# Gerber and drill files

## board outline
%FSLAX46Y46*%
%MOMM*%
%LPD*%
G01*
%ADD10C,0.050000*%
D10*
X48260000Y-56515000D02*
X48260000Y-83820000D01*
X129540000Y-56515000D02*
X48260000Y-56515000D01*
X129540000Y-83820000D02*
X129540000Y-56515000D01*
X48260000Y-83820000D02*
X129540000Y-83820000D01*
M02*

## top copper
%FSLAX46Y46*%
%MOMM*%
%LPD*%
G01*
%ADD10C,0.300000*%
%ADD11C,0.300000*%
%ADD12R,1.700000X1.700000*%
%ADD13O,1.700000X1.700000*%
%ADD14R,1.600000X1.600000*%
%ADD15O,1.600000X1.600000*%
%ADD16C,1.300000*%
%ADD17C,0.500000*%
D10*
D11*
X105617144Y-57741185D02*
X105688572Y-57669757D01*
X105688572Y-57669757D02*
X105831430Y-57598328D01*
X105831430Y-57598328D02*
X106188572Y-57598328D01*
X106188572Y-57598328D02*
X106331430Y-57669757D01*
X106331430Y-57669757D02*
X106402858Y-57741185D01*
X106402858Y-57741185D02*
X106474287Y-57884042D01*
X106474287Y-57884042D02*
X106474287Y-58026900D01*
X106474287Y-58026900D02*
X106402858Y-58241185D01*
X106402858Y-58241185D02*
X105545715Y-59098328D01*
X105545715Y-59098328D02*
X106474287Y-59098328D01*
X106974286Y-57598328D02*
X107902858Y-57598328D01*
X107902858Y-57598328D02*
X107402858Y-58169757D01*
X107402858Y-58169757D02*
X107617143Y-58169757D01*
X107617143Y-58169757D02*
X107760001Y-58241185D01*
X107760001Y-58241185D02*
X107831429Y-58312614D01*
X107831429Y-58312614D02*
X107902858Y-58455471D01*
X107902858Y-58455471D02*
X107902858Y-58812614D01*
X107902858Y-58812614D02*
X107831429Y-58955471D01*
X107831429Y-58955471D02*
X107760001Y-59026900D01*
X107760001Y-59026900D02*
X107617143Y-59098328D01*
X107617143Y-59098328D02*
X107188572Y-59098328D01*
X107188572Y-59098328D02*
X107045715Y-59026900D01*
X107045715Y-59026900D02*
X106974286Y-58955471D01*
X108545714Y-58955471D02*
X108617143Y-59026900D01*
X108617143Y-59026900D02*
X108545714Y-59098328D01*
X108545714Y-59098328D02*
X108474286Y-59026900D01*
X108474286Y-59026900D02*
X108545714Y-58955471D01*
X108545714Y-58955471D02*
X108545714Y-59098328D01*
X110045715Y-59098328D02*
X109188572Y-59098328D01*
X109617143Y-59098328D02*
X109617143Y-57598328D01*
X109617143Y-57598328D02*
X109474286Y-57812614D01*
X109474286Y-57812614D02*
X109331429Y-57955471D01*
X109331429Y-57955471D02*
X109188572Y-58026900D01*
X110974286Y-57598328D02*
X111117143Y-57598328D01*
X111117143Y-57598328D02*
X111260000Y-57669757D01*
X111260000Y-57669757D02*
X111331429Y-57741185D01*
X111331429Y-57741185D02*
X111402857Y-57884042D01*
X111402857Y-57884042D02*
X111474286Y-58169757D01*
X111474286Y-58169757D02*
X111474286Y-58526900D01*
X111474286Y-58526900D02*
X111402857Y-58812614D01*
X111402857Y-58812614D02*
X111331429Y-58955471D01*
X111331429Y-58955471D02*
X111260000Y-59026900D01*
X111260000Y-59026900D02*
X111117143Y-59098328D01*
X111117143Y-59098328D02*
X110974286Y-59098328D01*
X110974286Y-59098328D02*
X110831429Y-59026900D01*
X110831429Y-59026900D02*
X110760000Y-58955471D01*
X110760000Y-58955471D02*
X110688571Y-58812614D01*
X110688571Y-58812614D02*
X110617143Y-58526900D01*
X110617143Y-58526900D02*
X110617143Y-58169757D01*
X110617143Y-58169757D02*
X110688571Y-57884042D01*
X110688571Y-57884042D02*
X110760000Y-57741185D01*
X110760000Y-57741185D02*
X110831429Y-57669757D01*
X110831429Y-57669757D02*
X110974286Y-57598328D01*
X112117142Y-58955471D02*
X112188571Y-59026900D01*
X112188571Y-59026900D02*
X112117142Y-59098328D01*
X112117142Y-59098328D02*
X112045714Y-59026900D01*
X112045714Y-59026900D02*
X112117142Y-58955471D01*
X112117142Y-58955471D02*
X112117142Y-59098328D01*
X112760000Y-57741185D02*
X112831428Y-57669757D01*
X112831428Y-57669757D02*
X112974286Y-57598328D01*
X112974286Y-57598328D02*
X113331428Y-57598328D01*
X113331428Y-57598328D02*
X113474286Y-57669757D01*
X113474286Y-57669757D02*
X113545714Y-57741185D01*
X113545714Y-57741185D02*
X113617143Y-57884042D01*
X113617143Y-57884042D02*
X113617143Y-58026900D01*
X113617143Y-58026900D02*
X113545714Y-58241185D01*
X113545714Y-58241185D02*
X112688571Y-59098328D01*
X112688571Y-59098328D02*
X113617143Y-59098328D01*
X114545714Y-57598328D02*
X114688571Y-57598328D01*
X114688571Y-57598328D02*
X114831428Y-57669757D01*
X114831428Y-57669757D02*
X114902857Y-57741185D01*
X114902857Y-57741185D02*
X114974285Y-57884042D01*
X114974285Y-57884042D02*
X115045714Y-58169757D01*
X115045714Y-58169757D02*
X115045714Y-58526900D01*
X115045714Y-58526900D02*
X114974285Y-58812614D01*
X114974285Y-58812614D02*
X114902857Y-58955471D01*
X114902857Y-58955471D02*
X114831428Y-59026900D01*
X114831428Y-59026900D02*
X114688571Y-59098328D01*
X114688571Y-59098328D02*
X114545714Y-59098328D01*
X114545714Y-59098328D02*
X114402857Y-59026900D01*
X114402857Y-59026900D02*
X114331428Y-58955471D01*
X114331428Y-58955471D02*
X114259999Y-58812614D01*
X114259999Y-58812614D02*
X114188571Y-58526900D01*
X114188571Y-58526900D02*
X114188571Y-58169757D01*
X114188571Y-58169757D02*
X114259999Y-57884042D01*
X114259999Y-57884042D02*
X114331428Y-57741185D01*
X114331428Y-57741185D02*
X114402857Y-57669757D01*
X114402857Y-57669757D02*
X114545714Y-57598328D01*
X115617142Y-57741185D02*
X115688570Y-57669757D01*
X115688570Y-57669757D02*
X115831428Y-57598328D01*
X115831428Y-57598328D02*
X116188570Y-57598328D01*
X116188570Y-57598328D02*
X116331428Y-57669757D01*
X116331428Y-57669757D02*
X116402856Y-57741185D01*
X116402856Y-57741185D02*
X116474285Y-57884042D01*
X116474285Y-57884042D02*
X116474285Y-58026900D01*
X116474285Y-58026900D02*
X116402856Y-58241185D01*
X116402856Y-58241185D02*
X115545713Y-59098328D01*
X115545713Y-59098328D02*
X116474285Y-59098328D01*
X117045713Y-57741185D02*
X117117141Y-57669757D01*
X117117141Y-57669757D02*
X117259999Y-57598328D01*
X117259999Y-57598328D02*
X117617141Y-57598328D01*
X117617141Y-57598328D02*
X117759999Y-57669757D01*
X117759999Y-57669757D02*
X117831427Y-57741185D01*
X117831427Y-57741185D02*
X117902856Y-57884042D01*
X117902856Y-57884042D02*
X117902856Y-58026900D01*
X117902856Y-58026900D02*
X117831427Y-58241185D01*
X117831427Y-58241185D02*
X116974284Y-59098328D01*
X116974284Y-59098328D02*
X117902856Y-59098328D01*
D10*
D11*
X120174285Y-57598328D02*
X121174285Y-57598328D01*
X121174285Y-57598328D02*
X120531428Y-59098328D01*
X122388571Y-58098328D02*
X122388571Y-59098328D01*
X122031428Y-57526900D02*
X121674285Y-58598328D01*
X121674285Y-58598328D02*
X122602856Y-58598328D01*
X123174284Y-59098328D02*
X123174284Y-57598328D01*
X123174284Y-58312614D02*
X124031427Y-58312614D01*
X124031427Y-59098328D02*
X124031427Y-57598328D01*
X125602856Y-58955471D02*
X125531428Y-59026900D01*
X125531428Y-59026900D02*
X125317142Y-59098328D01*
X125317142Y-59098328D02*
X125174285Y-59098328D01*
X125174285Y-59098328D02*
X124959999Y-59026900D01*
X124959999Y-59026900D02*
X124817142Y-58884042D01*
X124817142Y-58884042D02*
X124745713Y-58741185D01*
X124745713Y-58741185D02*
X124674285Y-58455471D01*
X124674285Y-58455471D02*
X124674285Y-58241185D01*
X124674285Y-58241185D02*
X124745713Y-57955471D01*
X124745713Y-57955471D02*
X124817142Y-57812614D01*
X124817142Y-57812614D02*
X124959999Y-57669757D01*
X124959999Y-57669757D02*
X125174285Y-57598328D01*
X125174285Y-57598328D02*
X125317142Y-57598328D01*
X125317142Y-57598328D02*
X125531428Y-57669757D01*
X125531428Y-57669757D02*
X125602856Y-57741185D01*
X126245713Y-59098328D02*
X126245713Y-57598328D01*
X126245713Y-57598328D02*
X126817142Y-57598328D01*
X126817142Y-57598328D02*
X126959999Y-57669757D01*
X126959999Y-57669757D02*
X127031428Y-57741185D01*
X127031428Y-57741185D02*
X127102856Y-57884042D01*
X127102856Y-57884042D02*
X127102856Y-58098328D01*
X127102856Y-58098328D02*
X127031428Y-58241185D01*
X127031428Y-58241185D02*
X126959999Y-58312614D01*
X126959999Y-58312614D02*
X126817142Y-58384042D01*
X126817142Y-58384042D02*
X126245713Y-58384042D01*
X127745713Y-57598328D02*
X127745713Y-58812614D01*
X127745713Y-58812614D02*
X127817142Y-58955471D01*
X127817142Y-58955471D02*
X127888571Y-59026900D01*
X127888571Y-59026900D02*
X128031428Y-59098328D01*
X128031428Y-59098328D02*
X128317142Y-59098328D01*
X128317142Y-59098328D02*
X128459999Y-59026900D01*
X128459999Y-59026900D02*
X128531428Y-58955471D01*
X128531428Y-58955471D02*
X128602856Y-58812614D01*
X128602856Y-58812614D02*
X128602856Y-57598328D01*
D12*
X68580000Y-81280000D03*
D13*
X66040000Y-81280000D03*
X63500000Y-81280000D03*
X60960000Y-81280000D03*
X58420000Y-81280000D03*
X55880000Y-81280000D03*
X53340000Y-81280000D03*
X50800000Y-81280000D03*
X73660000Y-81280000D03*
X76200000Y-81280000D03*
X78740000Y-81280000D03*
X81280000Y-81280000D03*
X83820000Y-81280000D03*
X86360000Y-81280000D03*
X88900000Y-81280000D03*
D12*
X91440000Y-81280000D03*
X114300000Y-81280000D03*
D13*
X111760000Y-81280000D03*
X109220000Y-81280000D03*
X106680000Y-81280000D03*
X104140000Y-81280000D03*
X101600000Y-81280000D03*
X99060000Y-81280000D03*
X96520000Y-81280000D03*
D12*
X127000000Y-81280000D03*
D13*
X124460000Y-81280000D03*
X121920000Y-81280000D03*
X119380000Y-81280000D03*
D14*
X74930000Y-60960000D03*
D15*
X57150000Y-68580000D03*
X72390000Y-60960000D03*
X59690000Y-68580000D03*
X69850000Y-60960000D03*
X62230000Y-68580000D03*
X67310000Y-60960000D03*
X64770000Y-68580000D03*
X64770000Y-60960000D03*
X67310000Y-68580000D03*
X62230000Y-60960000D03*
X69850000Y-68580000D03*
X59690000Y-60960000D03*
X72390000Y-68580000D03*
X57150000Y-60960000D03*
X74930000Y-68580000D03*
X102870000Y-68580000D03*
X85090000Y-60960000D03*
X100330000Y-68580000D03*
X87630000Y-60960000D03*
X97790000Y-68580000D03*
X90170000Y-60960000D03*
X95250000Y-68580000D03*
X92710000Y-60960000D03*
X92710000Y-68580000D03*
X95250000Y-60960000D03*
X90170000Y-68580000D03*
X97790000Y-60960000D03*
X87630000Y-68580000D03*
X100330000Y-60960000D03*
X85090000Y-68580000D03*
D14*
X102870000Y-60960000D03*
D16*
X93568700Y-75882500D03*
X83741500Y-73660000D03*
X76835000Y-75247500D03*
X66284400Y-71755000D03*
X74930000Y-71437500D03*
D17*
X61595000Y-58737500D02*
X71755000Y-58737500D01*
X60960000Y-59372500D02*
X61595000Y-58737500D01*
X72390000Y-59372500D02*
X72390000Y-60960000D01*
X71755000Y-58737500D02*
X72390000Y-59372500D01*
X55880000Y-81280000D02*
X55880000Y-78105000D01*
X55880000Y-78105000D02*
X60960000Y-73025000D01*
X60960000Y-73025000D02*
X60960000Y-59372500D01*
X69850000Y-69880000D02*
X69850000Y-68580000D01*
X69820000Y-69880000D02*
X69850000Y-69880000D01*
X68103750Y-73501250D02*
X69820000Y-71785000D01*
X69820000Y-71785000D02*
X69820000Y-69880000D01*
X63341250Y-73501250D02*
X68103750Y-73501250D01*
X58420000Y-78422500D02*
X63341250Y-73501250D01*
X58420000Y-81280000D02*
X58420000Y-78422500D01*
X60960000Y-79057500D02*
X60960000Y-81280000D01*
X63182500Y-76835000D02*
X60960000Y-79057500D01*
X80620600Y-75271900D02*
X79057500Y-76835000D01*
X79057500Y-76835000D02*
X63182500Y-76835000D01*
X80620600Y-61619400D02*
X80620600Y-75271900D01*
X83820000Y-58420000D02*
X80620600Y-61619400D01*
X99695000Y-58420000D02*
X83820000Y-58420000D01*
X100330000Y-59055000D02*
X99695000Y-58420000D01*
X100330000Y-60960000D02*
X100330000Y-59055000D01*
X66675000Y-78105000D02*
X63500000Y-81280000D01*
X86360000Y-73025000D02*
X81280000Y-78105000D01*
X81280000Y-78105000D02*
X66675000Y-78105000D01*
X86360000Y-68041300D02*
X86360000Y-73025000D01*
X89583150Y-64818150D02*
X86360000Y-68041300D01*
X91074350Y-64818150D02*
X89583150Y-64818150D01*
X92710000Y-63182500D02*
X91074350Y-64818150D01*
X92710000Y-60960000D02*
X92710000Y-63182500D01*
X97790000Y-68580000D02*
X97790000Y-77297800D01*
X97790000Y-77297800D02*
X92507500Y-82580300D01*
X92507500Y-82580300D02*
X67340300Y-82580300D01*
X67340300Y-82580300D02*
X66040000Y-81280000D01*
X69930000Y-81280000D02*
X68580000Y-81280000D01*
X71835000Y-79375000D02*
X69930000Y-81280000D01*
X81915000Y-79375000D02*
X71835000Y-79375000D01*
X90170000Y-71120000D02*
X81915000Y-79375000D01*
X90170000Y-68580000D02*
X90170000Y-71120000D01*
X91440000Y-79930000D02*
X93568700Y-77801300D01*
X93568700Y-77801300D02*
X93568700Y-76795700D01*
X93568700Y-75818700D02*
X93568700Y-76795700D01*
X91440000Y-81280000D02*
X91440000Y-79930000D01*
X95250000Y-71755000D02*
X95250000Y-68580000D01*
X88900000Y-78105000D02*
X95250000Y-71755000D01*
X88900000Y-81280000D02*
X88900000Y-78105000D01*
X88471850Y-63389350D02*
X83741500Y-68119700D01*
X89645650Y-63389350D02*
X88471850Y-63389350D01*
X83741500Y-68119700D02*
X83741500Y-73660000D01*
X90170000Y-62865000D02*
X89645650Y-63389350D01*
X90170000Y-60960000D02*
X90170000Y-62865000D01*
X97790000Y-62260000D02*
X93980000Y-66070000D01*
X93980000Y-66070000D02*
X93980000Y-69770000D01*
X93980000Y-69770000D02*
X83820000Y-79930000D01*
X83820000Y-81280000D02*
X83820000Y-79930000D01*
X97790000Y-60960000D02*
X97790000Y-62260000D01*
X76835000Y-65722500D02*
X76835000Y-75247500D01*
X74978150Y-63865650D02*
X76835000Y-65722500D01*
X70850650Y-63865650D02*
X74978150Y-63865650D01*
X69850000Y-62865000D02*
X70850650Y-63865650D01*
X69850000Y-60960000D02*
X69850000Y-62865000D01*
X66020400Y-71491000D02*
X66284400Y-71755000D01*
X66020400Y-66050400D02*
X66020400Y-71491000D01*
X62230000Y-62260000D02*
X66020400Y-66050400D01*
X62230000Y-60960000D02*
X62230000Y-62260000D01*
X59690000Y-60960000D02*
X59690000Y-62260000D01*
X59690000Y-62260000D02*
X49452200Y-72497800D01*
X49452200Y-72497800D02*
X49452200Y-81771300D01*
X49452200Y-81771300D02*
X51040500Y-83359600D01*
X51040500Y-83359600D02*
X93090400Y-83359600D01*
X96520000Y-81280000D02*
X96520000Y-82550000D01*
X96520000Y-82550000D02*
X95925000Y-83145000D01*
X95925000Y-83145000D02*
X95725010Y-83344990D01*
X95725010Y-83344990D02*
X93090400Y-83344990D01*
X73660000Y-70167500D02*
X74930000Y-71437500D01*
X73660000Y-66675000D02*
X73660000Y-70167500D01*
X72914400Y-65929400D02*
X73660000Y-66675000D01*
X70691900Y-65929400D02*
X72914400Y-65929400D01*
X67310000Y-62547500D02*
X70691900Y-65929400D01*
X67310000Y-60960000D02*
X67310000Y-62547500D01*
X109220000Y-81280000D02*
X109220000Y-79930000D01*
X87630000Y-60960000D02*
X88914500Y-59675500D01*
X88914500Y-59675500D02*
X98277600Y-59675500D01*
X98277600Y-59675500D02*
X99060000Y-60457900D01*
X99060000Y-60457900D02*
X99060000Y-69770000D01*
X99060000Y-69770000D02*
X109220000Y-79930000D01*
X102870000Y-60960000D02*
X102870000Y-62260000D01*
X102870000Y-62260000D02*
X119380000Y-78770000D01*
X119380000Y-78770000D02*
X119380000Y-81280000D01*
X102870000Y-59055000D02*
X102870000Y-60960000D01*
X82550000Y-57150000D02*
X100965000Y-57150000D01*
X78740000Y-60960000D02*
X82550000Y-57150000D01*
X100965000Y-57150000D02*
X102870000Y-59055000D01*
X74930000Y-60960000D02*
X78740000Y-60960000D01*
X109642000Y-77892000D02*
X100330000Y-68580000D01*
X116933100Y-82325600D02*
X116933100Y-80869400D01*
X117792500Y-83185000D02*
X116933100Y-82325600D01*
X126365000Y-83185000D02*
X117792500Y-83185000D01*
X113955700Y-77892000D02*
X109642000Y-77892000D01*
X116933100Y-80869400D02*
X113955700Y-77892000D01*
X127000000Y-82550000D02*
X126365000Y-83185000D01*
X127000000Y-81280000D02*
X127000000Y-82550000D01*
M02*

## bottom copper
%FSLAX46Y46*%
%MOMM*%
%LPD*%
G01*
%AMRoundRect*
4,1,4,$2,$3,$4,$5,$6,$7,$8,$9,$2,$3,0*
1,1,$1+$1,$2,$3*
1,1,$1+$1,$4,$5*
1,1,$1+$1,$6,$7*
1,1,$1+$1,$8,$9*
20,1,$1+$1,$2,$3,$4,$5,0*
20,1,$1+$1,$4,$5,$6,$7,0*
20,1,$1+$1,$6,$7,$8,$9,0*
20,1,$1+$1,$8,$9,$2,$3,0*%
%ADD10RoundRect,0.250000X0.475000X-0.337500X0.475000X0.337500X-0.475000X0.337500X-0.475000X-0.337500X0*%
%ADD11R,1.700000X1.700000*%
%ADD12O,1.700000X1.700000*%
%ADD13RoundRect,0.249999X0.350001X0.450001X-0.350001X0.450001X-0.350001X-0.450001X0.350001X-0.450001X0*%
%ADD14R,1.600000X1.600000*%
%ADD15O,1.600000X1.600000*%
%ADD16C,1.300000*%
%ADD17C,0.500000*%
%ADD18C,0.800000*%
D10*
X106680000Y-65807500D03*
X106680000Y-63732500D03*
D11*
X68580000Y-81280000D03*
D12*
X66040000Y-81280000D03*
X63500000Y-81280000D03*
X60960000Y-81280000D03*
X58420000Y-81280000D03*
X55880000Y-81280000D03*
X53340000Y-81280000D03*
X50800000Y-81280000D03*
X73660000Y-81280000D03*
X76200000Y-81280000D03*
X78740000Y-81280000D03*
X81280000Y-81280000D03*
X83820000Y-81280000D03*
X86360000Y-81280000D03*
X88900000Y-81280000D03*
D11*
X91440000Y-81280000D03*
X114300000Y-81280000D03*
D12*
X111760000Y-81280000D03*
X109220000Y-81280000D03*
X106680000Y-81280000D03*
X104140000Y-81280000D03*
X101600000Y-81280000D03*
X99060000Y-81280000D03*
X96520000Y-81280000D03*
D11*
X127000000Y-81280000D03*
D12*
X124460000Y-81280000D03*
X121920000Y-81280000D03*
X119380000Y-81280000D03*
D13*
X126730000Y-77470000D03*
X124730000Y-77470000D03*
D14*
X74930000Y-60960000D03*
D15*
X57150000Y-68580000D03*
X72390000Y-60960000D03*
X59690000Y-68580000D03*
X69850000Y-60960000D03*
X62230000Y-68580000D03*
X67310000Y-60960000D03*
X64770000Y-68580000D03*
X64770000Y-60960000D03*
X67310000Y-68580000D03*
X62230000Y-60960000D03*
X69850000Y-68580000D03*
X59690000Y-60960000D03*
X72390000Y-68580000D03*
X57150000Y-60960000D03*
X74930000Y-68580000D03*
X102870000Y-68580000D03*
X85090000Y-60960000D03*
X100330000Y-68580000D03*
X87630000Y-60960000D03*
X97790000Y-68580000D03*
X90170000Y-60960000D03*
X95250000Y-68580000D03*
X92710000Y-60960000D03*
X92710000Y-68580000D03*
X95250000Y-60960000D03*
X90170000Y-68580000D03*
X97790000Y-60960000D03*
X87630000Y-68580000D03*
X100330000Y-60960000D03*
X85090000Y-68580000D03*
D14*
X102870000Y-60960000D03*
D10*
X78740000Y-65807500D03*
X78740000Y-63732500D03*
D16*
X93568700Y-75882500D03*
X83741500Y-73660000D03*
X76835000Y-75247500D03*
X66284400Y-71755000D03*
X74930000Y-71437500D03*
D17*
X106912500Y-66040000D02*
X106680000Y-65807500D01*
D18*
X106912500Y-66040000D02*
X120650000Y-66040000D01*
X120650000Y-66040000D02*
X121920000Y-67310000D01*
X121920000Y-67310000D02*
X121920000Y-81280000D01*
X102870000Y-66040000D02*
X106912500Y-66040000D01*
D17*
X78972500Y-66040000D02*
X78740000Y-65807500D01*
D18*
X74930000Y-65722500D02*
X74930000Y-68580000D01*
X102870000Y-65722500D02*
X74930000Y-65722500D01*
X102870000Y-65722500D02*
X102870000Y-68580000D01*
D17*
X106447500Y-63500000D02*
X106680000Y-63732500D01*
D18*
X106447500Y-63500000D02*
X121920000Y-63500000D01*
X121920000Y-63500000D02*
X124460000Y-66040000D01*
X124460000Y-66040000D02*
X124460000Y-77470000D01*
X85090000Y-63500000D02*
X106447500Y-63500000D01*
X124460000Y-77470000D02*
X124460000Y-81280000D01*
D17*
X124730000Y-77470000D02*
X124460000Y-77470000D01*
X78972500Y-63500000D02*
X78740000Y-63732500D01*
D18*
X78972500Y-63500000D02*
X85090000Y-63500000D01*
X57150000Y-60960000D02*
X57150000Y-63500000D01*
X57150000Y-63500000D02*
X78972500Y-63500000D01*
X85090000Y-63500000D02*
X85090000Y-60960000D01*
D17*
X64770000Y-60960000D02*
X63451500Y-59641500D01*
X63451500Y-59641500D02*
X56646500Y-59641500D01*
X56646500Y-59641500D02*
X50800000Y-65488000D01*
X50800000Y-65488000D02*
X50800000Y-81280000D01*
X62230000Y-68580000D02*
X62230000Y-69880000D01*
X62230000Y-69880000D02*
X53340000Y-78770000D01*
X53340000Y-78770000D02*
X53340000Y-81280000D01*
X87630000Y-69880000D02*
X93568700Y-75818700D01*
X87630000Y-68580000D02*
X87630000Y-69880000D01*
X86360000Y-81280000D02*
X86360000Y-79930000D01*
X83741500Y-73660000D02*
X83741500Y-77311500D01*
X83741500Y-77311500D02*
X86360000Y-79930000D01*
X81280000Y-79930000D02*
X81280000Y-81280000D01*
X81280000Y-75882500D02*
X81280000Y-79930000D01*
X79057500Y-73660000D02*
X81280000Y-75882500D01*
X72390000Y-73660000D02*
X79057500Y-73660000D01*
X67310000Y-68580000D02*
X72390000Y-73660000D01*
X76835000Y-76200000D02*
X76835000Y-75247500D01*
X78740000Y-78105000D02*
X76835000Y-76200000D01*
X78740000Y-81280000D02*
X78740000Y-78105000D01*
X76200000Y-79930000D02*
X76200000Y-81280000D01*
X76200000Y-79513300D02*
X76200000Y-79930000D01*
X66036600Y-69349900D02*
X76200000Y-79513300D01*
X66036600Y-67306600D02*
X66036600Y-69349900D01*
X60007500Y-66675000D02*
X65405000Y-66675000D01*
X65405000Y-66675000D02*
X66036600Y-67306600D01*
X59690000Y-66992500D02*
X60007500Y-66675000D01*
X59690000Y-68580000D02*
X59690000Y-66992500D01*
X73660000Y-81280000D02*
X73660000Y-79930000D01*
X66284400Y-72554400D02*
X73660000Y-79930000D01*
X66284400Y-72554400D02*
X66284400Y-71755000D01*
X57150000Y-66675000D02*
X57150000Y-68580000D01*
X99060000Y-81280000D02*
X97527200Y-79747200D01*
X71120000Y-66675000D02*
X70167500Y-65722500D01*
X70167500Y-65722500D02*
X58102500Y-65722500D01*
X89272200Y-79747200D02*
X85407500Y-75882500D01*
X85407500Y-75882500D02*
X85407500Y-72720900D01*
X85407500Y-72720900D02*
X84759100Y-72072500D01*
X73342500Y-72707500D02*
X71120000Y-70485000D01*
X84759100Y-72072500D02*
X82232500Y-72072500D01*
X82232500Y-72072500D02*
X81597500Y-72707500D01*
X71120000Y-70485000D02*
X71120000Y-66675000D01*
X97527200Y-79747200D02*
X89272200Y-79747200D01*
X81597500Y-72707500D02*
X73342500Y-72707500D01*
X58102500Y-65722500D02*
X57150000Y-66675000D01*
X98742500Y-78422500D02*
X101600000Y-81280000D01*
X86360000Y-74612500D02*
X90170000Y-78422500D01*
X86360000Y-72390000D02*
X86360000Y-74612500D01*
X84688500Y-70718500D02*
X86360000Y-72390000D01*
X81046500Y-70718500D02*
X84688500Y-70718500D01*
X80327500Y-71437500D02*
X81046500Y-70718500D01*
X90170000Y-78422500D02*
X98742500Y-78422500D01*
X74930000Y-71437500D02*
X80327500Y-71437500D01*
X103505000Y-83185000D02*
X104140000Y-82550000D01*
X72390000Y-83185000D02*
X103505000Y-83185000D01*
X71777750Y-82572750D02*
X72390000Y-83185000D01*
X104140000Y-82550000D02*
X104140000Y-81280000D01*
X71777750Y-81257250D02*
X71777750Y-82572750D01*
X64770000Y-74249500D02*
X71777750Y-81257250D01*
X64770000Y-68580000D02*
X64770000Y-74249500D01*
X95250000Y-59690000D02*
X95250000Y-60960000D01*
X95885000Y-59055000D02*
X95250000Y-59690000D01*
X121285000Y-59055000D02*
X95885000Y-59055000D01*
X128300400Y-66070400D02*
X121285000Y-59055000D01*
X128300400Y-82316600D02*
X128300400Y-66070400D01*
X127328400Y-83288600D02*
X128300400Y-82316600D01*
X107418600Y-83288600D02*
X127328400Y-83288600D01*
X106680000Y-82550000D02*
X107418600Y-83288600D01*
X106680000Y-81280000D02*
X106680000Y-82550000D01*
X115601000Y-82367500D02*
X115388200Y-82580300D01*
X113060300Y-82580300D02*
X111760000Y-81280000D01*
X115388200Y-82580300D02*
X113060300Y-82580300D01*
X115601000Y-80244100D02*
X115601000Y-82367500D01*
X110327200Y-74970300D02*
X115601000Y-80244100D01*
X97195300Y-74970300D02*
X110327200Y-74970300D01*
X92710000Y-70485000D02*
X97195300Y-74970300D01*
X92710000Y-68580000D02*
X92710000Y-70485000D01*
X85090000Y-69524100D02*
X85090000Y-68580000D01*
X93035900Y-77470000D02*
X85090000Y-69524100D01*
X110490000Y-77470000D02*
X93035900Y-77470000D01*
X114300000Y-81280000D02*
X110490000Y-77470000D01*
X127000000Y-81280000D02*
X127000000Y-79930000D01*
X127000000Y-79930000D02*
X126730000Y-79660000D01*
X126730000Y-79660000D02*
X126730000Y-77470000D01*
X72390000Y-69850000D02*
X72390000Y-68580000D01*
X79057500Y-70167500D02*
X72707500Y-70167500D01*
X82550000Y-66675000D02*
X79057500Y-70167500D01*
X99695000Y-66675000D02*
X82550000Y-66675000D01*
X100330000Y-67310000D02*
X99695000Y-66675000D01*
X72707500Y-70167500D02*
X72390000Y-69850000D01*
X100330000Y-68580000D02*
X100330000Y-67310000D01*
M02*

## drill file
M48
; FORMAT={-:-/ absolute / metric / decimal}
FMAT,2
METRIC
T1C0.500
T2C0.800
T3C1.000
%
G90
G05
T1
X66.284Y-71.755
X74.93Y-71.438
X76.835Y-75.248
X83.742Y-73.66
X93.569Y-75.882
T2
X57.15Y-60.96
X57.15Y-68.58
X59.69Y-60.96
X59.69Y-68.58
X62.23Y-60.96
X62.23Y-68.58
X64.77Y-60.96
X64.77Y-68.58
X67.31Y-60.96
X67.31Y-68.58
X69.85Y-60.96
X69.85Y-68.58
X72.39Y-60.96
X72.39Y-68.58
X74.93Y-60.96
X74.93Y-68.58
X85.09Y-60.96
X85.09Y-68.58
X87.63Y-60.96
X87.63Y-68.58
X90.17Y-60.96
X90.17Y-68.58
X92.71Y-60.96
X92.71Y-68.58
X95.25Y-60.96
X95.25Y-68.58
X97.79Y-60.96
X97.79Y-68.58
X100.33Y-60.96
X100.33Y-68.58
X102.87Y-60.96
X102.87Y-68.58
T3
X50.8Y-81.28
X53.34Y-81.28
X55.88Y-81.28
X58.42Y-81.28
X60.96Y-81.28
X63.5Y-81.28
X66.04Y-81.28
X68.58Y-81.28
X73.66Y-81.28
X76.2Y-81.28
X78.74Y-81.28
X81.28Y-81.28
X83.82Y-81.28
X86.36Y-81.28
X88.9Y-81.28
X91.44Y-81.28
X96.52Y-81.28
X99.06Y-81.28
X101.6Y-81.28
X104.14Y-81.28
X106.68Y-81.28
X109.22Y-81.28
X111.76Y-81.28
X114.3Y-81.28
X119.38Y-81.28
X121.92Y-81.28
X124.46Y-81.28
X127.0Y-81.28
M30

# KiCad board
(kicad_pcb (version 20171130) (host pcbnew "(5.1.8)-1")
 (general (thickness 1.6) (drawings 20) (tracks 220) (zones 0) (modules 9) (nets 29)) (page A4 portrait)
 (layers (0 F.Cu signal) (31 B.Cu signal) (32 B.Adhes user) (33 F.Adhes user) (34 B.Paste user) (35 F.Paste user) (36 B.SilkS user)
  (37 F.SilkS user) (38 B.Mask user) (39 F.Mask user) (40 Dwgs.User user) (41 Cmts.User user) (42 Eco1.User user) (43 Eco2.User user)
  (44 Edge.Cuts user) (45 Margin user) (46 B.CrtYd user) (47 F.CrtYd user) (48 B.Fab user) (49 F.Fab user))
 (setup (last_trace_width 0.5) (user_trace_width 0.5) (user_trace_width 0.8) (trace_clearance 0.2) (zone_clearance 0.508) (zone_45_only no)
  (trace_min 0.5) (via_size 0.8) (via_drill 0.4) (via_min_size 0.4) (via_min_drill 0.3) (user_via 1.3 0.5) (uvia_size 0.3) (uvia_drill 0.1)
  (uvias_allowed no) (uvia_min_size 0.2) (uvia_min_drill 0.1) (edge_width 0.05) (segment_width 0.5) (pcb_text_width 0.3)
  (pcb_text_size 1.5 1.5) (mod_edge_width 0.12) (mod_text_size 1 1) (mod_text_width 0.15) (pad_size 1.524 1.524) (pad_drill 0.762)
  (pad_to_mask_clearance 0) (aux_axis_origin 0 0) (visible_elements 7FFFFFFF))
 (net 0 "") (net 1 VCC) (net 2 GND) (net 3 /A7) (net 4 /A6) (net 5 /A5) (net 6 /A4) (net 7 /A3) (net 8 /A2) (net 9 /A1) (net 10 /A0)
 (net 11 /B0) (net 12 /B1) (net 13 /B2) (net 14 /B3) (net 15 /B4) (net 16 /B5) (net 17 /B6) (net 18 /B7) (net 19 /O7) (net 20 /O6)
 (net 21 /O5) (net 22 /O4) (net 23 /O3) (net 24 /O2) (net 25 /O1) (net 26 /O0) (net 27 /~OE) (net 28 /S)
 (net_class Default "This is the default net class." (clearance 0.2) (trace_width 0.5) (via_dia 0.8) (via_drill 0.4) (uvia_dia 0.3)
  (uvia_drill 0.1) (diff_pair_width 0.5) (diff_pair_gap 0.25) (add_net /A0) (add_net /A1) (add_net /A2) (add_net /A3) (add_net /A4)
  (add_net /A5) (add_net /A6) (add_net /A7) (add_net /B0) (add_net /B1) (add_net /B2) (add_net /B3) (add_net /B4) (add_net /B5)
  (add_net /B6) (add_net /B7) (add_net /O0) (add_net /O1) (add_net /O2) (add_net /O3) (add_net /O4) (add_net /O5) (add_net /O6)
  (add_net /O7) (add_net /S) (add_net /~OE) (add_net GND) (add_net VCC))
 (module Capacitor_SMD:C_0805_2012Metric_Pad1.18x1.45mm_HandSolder (layer B.Cu) (at 106.68 64.77 90)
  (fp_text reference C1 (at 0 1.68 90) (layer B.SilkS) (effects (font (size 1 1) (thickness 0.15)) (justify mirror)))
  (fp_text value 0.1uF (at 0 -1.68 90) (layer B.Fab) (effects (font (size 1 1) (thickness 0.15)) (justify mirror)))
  (pad 1 smd roundrect (at -1.0375 0 90) (size 1.175 1.45) (layers B.Cu B.Paste B.Mask) (roundrect_rratio 0.2127659574468085) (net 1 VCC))
  (pad 2 smd roundrect (at 1.0375 0 90) (size 1.175 1.45) (layers B.Cu B.Paste B.Mask) (roundrect_rratio 0.2127659574468085) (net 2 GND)))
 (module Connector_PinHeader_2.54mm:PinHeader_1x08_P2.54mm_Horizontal (layer F.Cu) (at 68.58 81.28 270)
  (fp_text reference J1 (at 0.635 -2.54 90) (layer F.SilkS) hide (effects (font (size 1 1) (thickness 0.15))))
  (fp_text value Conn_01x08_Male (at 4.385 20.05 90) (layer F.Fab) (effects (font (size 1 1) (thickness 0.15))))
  (pad 1 thru_hole rect (at 0 0 270) (size 1.7 1.7) (drill 1) (layers *.Cu *.Mask) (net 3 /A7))
  (pad 2 thru_hole oval (at 0 2.54 270) (size 1.7 1.7) (drill 1) (layers *.Cu *.Mask) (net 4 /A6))
  (pad 3 thru_hole oval (at 0 5.08 270) (size 1.7 1.7) (drill 1) (layers *.Cu *.Mask) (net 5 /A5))
  (pad 4 thru_hole oval (at 0 7.62 270) (size 1.7 1.7) (drill 1) (layers *.Cu *.Mask) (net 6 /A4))
  (pad 5 thru_hole oval (at 0 10.16 270) (size 1.7 1.7) (drill 1) (layers *.Cu *.Mask) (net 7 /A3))
  (pad 6 thru_hole oval (at 0 12.7 270) (size 1.7 1.7) (drill 1) (layers *.Cu *.Mask) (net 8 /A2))
  (pad 7 thru_hole oval (at 0 15.24 270) (size 1.7 1.7) (drill 1) (layers *.Cu *.Mask) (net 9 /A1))
  (pad 8 thru_hole oval (at 0 17.78 270) (size 1.7 1.7) (drill 1) (layers *.Cu *.Mask) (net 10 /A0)))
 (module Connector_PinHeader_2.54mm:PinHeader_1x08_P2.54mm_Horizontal (layer F.Cu) (at 91.44 81.28 270)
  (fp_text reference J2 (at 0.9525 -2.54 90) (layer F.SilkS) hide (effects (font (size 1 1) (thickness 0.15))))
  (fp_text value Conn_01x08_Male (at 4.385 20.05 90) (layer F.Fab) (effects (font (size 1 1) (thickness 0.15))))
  (pad 8 thru_hole oval (at 0 17.78 270) (size 1.7 1.7) (drill 1) (layers *.Cu *.Mask) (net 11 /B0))
  (pad 7 thru_hole oval (at 0 15.24 270) (size 1.7 1.7) (drill 1) (layers *.Cu *.Mask) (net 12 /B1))
  (pad 6 thru_hole oval (at 0 12.7 270) (size 1.7 1.7) (drill 1) (layers *.Cu *.Mask) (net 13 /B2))
  (pad 5 thru_hole oval (at 0 10.16 270) (size 1.7 1.7) (drill 1) (layers *.Cu *.Mask) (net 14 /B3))
  (pad 4 thru_hole oval (at 0 7.62 270) (size 1.7 1.7) (drill 1) (layers *.Cu *.Mask) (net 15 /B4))
  (pad 3 thru_hole oval (at 0 5.08 270) (size 1.7 1.7) (drill 1) (layers *.Cu *.Mask) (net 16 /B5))
  (pad 2 thru_hole oval (at 0 2.54 270) (size 1.7 1.7) (drill 1) (layers *.Cu *.Mask) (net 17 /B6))
  (pad 1 thru_hole rect (at 0 0 270) (size 1.7 1.7) (drill 1) (layers *.Cu *.Mask) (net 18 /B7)))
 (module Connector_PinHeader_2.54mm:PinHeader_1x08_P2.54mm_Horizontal (layer F.Cu) (at 114.3 81.28 270)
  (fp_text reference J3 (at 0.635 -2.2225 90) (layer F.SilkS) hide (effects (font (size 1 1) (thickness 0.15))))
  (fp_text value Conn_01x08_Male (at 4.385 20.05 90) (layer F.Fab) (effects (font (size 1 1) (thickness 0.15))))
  (pad 1 thru_hole rect (at 0 0 270) (size 1.7 1.7) (drill 1) (layers *.Cu *.Mask) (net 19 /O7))
  (pad 2 thru_hole oval (at 0 2.54 270) (size 1.7 1.7) (drill 1) (layers *.Cu *.Mask) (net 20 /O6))
  (pad 3 thru_hole oval (at 0 5.08 270) (size 1.7 1.7) (drill 1) (layers *.Cu *.Mask) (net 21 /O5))
  (pad 4 thru_hole oval (at 0 7.62 270) (size 1.7 1.7) (drill 1) (layers *.Cu *.Mask) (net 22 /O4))
  (pad 5 thru_hole oval (at 0 10.16 270) (size 1.7 1.7) (drill 1) (layers *.Cu *.Mask) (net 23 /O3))
  (pad 6 thru_hole oval (at 0 12.7 270) (size 1.7 1.7) (drill 1) (layers *.Cu *.Mask) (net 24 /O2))
  (pad 7 thru_hole oval (at 0 15.24 270) (size 1.7 1.7) (drill 1) (layers *.Cu *.Mask) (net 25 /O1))
  (pad 8 thru_hole oval (at 0 17.78 270) (size 1.7 1.7) (drill 1) (layers *.Cu *.Mask) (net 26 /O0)))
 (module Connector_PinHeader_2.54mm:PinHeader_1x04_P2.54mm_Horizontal (layer F.Cu) (at 127 81.28 270)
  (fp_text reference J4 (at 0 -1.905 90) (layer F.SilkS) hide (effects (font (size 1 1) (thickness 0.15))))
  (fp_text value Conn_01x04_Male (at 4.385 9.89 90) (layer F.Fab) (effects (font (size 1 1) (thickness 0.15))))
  (pad 1 thru_hole rect (at 0 0 270) (size 1.7 1.7) (drill 1) (layers *.Cu *.Mask) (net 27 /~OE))
  (pad 2 thru_hole oval (at 0 2.54 270) (size 1.7 1.7) (drill 1) (layers *.Cu *.Mask) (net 2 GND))
  (pad 3 thru_hole oval (at 0 5.08 270) (size 1.7 1.7) (drill 1) (layers *.Cu *.Mask) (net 1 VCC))
  (pad 4 thru_hole oval (at 0 7.62 270) (size 1.7 1.7) (drill 1) (layers *.Cu *.Mask) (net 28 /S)))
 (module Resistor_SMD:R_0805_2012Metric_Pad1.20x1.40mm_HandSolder (layer B.Cu) (at 125.73 77.47 180)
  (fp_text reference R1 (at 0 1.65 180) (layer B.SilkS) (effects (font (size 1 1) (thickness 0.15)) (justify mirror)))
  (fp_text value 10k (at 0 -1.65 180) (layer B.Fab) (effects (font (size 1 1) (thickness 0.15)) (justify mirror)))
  (pad 1 smd roundrect (at -1 0 180) (size 1.2 1.4) (layers B.Cu B.Paste B.Mask) (roundrect_rratio 0.2083325) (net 27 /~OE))
  (pad 2 smd roundrect (at 1 0 180) (size 1.2 1.4) (layers B.Cu B.Paste B.Mask) (roundrect_rratio 0.2083325) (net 2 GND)))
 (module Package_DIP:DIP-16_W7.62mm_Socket (layer F.Cu) (at 74.93 60.96 270)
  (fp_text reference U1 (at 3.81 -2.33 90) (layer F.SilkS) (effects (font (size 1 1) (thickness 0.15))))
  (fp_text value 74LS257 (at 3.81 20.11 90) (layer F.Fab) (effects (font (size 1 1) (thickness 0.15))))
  (pad 1 thru_hole rect (at 0 0 270) (size 1.6 1.6) (drill 0.8) (layers *.Cu *.Mask) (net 28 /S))
  (pad 9 thru_hole oval (at 7.62 17.78 270) (size 1.6 1.6) (drill 0.8) (layers *.Cu *.Mask) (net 25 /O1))
  (pad 2 thru_hole oval (at 0 2.54 270) (size 1.6 1.6) (drill 0.8) (layers *.Cu *.Mask) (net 8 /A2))
  (pad 10 thru_hole oval (at 7.62 15.24 270) (size 1.6 1.6) (drill 0.8) (layers *.Cu *.Mask) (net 12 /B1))
  (pad 3 thru_hole oval (at 0 5.08 270) (size 1.6 1.6) (drill 0.8) (layers *.Cu *.Mask) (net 13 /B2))
  (pad 11 thru_hole oval (at 7.62 12.7 270) (size 1.6 1.6) (drill 0.8) (layers *.Cu *.Mask) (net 9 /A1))
  (pad 4 thru_hole oval (at 0 7.62 270) (size 1.6 1.6) (drill 0.8) (layers *.Cu *.Mask) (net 24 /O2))
  (pad 12 thru_hole oval (at 7.62 10.16 270) (size 1.6 1.6) (drill 0.8) (layers *.Cu *.Mask) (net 23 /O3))
  (pad 5 thru_hole oval (at 0 10.16 270) (size 1.6 1.6) (drill 0.8) (layers *.Cu *.Mask) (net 10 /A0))
  (pad 13 thru_hole oval (at 7.62 7.62 270) (size 1.6 1.6) (drill 0.8) (layers *.Cu *.Mask) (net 14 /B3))
  (pad 6 thru_hole oval (at 0 12.7 270) (size 1.6 1.6) (drill 0.8) (layers *.Cu *.Mask) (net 11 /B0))
  (pad 14 thru_hole oval (at 7.62 5.08 270) (size 1.6 1.6) (drill 0.8) (layers *.Cu *.Mask) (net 7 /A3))
  (pad 7 thru_hole oval (at 0 15.24 270) (size 1.6 1.6) (drill 0.8) (layers *.Cu *.Mask) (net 26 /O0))
  (pad 15 thru_hole oval (at 7.62 2.54 270) (size 1.6 1.6) (drill 0.8) (layers *.Cu *.Mask) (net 27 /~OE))
  (pad 8 thru_hole oval (at 0 17.78 270) (size 1.6 1.6) (drill 0.8) (layers *.Cu *.Mask) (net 2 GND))
  (pad 16 thru_hole oval (at 7.62 0 270) (size 1.6 1.6) (drill 0.8) (layers *.Cu *.Mask) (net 1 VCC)))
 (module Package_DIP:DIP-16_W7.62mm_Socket (layer F.Cu) (at 102.87 60.96 270)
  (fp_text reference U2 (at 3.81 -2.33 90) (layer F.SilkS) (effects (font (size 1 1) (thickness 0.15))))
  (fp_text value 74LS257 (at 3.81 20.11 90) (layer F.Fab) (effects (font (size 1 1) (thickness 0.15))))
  (pad 16 thru_hole oval (at 7.62 0 270) (size 1.6 1.6) (drill 0.8) (layers *.Cu *.Mask) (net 1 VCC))
  (pad 8 thru_hole oval (at 0 17.78 270) (size 1.6 1.6) (drill 0.8) (layers *.Cu *.Mask) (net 2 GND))
  (pad 15 thru_hole oval (at 7.62 2.54 270) (size 1.6 1.6) (drill 0.8) (layers *.Cu *.Mask) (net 27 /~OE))
  (pad 7 thru_hole oval (at 0 15.24 270) (size 1.6 1.6) (drill 0.8) (layers *.Cu *.Mask) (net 21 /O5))
  (pad 14 thru_hole oval (at 7.62 5.08 270) (size 1.6 1.6) (drill 0.8) (layers *.Cu *.Mask) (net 4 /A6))
  (pad 6 thru_hole oval (at 0 12.7 270) (size 1.6 1.6) (drill 0.8) (layers *.Cu *.Mask) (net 16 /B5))
  (pad 13 thru_hole oval (at 7.62 7.62 270) (size 1.6 1.6) (drill 0.8) (layers *.Cu *.Mask) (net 17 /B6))
  (pad 5 thru_hole oval (at 0 10.16 270) (size 1.6 1.6) (drill 0.8) (layers *.Cu *.Mask) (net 5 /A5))
  (pad 12 thru_hole oval (at 7.62 10.16 270) (size 1.6 1.6) (drill 0.8) (layers *.Cu *.Mask) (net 20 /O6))
  (pad 4 thru_hole oval (at 0 7.62 270) (size 1.6 1.6) (drill 0.8) (layers *.Cu *.Mask) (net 22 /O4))
  (pad 11 thru_hole oval (at 7.62 12.7 270) (size 1.6 1.6) (drill 0.8) (layers *.Cu *.Mask) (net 3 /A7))
  (pad 3 thru_hole oval (at 0 5.08 270) (size 1.6 1.6) (drill 0.8) (layers *.Cu *.Mask) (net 15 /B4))
  (pad 10 thru_hole oval (at 7.62 15.24 270) (size 1.6 1.6) (drill 0.8) (layers *.Cu *.Mask) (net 18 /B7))
  (pad 2 thru_hole oval (at 0 2.54 270) (size 1.6 1.6) (drill 0.8) (layers *.Cu *.Mask) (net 6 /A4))
  (pad 9 thru_hole oval (at 7.62 17.78 270) (size 1.6 1.6) (drill 0.8) (layers *.Cu *.Mask) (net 19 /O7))
  (pad 1 thru_hole rect (at 0 0 270) (size 1.6 1.6) (drill 0.8) (layers *.Cu *.Mask) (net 28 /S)))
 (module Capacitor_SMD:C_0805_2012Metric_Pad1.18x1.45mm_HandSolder (layer B.Cu) (at 78.74 64.77 90)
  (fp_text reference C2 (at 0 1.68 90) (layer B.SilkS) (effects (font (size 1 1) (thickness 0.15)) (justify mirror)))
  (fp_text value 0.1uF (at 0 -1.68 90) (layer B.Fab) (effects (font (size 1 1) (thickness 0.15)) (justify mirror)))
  (pad 1 smd roundrect (at -1.0375 0 90) (size 1.175 1.45) (layers B.Cu B.Paste B.Mask) (roundrect_rratio 0.2127659574468085) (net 1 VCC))
  (pad 2 smd roundrect (at 1.0375 0 90) (size 1.175 1.45) (layers B.Cu B.Paste B.Mask) (roundrect_rratio 0.2127659574468085) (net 2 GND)))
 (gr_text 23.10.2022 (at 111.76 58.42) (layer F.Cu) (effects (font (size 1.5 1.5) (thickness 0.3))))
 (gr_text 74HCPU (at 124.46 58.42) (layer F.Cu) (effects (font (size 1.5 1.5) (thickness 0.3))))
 (gr_line (start 48.26 56.515) (end 48.26 83.82) (layer Edge.Cuts) (width 0.05))
 (gr_line (start 129.54 56.515) (end 48.26 56.515) (layer Edge.Cuts) (width 0.05))
 (gr_line (start 129.54 83.82) (end 129.54 56.515) (layer Edge.Cuts) (width 0.05))
 (gr_line (start 48.26 83.82) (end 129.54 83.82) (layer Edge.Cuts) (width 0.05))
 (segment (start 106.9125 66.04) (end 106.68 65.8075) (width 0.5) (layer B.Cu) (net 1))
 (segment (start 106.9125 66.04) (end 120.65 66.04) (width 0.8) (layer B.Cu) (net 1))
 (segment (start 120.65 66.04) (end 121.92 67.31) (width 0.8) (layer B.Cu) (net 1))
 (segment (start 121.92 67.31) (end 121.92 81.28) (width 0.8) (layer B.Cu) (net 1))
 (segment (start 102.87 66.04) (end 106.9125 66.04) (width 0.8) (layer B.Cu) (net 1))
 (segment (start 78.9725 66.04) (end 78.74 65.8075) (width 0.5) (layer B.Cu) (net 1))
 (segment (start 74.93 65.7225) (end 74.93 68.58) (width 0.8) (layer B.Cu) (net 1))
 (segment (start 102.87 65.7225) (end 74.93 65.7225) (width 0.8) (layer B.Cu) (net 1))
 (segment (start 102.87 65.7225) (end 102.87 68.58) (width 0.8) (layer B.Cu) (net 1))
 (segment (start 106.4475 63.5) (end 106.68 63.7325) (width 0.5) (layer B.Cu) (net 2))
 (segment (start 106.4475 63.5) (end 121.92 63.5) (width 0.8) (layer B.Cu) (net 2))
 (segment (start 121.92 63.5) (end 124.46 66.04) (width 0.8) (layer B.Cu) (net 2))
 (segment (start 124.46 66.04) (end 124.46 77.47) (width 0.8) (layer B.Cu) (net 2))
 (segment (start 85.09 63.5) (end 106.4475 63.5) (width 0.8) (layer B.Cu) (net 2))
 (segment (start 124.46 77.47) (end 124.46 81.28) (width 0.8) (layer B.Cu) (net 2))
 (segment (start 124.73 77.47) (end 124.46 77.47) (width 0.5) (layer B.Cu) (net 2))
 (segment (start 78.9725 63.5) (end 78.74 63.7325) (width 0.5) (layer B.Cu) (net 2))
 (segment (start 78.9725 63.5) (end 85.09 63.5) (width 0.8) (layer B.Cu) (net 2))
 (segment (start 57.15 60.96) (end 57.15 63.5) (width 0.8) (layer B.Cu) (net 2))
 (segment (start 57.15 63.5) (end 78.9725 63.5) (width 0.8) (layer B.Cu) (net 2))
 (segment (start 85.09 63.5) (end 85.09 60.96) (width 0.8) (layer B.Cu) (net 2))
 (segment (start 64.77 60.96) (end 63.4515 59.6415) (width 0.5) (layer B.Cu) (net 10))
 (segment (start 63.4515 59.6415) (end 56.6465 59.6415) (width 0.5) (layer B.Cu) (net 10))
 (segment (start 56.6465 59.6415) (end 50.8 65.488) (width 0.5) (layer B.Cu) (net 10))
 (segment (start 50.8 65.488) (end 50.8 81.28) (width 0.5) (layer B.Cu) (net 10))
 (segment (start 62.23 68.58) (end 62.23 69.88) (width 0.5) (layer B.Cu) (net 9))
 (segment (start 62.23 69.88) (end 53.34 78.77) (width 0.5) (layer B.Cu) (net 9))
 (segment (start 53.34 78.77) (end 53.34 81.28) (width 0.5) (layer B.Cu) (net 9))
 (segment (start 61.595 58.7375) (end 71.755 58.7375) (width 0.5) (layer F.Cu) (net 8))
 (segment (start 60.96 59.3725) (end 61.595 58.7375) (width 0.5) (layer F.Cu) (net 8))
 (segment (start 72.39 59.3725) (end 72.39 60.96) (width 0.5) (layer F.Cu) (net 8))
 (segment (start 71.755 58.7375) (end 72.39 59.3725) (width 0.5) (layer F.Cu) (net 8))
 (segment (start 55.88 81.28) (end 55.88 78.105) (width 0.5) (layer F.Cu) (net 8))
 (segment (start 55.88 78.105) (end 60.96 73.025) (width 0.5) (layer F.Cu) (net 8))
 (segment (start 60.96 73.025) (end 60.96 59.3725) (width 0.5) (layer F.Cu) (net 8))
 (segment (start 69.85 69.88) (end 69.85 68.58) (width 0.5) (layer F.Cu) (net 7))
 (segment (start 69.82 69.88) (end 69.85 69.88) (width 0.5) (layer F.Cu) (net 7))
 (segment (start 68.10375 73.50125) (end 69.82 71.785) (width 0.5) (layer F.Cu) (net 7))
 (segment (start 69.82 71.785) (end 69.82 69.88) (width 0.5) (layer F.Cu) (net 7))
 (segment (start 63.34125 73.50125) (end 68.10375 73.50125) (width 0.5) (layer F.Cu) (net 7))
 (segment (start 58.42 78.4225) (end 63.34125 73.50125) (width 0.5) (layer F.Cu) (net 7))
 (segment (start 58.42 81.28) (end 58.42 78.4225) (width 0.5) (layer F.Cu) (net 7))
 (segment (start 60.96 79.0575) (end 60.96 81.28) (width 0.5) (layer F.Cu) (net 6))
 (segment (start 63.1825 76.835) (end 60.96 79.0575) (width 0.5) (layer F.Cu) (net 6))
 (segment (start 80.6206 75.2719) (end 79.0575 76.835) (width 0.5) (layer F.Cu) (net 6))
 (segment (start 79.0575 76.835) (end 63.1825 76.835) (width 0.5) (layer F.Cu) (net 6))
 (segment (start 80.6206 61.6194) (end 80.6206 75.2719) (width 0.5) (layer F.Cu) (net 6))
 (segment (start 83.82 58.42) (end 80.6206 61.6194) (width 0.5) (layer F.Cu) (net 6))
 (segment (start 99.695 58.42) (end 83.82 58.42) (width 0.5) (layer F.Cu) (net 6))
 (segment (start 100.33 59.055) (end 99.695 58.42) (width 0.5) (layer F.Cu) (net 6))
 (segment (start 100.33 60.96) (end 100.33 59.055) (width 0.5) (layer F.Cu) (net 6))
 (segment (start 66.675 78.105) (end 63.5 81.28) (width 0.5) (layer F.Cu) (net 5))
 (segment (start 86.36 73.025) (end 81.28 78.105) (width 0.5) (layer F.Cu) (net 5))
 (segment (start 81.28 78.105) (end 66.675 78.105) (width 0.5) (layer F.Cu) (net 5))
 (segment (start 86.36 68.0413) (end 86.36 73.025) (width 0.5) (layer F.Cu) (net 5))
 (segment (start 89.58315 64.81815) (end 86.36 68.0413) (width 0.5) (layer F.Cu) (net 5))
 (segment (start 91.07435 64.81815) (end 89.58315 64.81815) (width 0.5) (layer F.Cu) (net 5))
 (segment (start 92.71 63.1825) (end 91.07435 64.81815) (width 0.5) (layer F.Cu) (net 5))
 (segment (start 92.71 60.96) (end 92.71 63.1825) (width 0.5) (layer F.Cu) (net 5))
 (segment (start 97.79 68.58) (end 97.79 77.2978) (width 0.5) (layer F.Cu) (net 4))
 (segment (start 97.79 77.2978) (end 92.5075 82.5803) (width 0.5) (layer F.Cu) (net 4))
 (segment (start 92.5075 82.5803) (end 67.3403 82.5803) (width 0.5) (layer F.Cu) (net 4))
 (segment (start 67.3403 82.5803) (end 66.04 81.28) (width 0.5) (layer F.Cu) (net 4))
 (segment (start 69.93 81.28) (end 68.58 81.28) (width 0.5) (layer F.Cu) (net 3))
 (segment (start 71.835 79.375) (end 69.93 81.28) (width 0.5) (layer F.Cu) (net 3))
 (segment (start 81.915 79.375) (end 71.835 79.375) (width 0.5) (layer F.Cu) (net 3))
 (segment (start 90.17 71.12) (end 81.915 79.375) (width 0.5) (layer F.Cu) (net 3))
 (segment (start 90.17 68.58) (end 90.17 71.12) (width 0.5) (layer F.Cu) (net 3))
 (segment (start 91.44 79.93) (end 93.5687 77.8013) (width 0.5) (layer F.Cu) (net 18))
 (segment (start 93.5687 77.8013) (end 93.5687 76.7957) (width 0.5) (layer F.Cu) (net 18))
 (segment (start 87.63 69.88) (end 93.5687 75.8187) (width 0.5) (layer B.Cu) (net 18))
 (segment (start 93.5687 75.8187) (end 93.5687 76.7957) (width 0.5) (layer F.Cu) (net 18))
 (segment (start 87.63 68.58) (end 87.63 69.88) (width 0.5) (layer B.Cu) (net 18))
 (segment (start 91.44 81.28) (end 91.44 79.93) (width 0.5) (layer F.Cu) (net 18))
 (via (at 93.5687 75.8825) (size 1.3) (drill 0.5) (layers F.Cu B.Cu) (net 18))
 (segment (start 95.25 71.755) (end 95.25 68.58) (width 0.5) (layer F.Cu) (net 17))
 (segment (start 88.9 78.105) (end 95.25 71.755) (width 0.5) (layer F.Cu) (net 17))
 (segment (start 88.9 81.28) (end 88.9 78.105) (width 0.5) (layer F.Cu) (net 17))
 (segment (start 86.36 81.28) (end 86.36 79.93) (width 0.5) (layer B.Cu) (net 16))
 (segment (start 83.7415 73.66) (end 83.7415 77.3115) (width 0.5) (layer B.Cu) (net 16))
 (segment (start 83.7415 77.3115) (end 86.36 79.93) (width 0.5) (layer B.Cu) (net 16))
 (via (at 83.7415 73.66) (size 1.3) (drill 0.5) (layers F.Cu B.Cu) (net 16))
 (segment (start 88.47185 63.38935) (end 83.7415 68.1197) (width 0.5) (layer F.Cu) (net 16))
 (segment (start 89.64565 63.38935) (end 88.47185 63.38935) (width 0.5) (layer F.Cu) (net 16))
 (segment (start 83.7415 68.1197) (end 83.7415 73.66) (width 0.5) (layer F.Cu) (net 16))
 (segment (start 90.17 62.865) (end 89.64565 63.38935) (width 0.5) (layer F.Cu) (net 16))
 (segment (start 90.17 60.96) (end 90.17 62.865) (width 0.5) (layer F.Cu) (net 16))
 (segment (start 97.79 62.26) (end 93.98 66.07) (width 0.5) (layer F.Cu) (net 15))
 (segment (start 93.98 66.07) (end 93.98 69.77) (width 0.5) (layer F.Cu) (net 15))
 (segment (start 93.98 69.77) (end 83.82 79.93) (width 0.5) (layer F.Cu) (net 15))
 (segment (start 83.82 81.28) (end 83.82 79.93) (width 0.5) (layer F.Cu) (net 15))
 (segment (start 97.79 60.96) (end 97.79 62.26) (width 0.5) (layer F.Cu) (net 15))
 (segment (start 81.28 79.93) (end 81.28 81.28) (width 0.5) (layer B.Cu) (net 14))
 (segment (start 81.28 75.8825) (end 81.28 79.93) (width 0.5) (layer B.Cu) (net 14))
 (segment (start 79.0575 73.66) (end 81.28 75.8825) (width 0.5) (layer B.Cu) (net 14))
 (segment (start 72.39 73.66) (end 79.0575 73.66) (width 0.5) (layer B.Cu) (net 14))
 (segment (start 67.31 68.58) (end 72.39 73.66) (width 0.5) (layer B.Cu) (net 14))
 (via (at 76.835 75.2475) (size 1.3) (drill 0.5) (layers F.Cu B.Cu) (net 13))
 (segment (start 76.835 76.2) (end 76.835 75.2475) (width 0.5) (layer B.Cu) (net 13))
 (segment (start 78.74 78.105) (end 76.835 76.2) (width 0.5) (layer B.Cu) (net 13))
 (segment (start 78.74 81.28) (end 78.74 78.105) (width 0.5) (layer B.Cu) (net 13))
 (segment (start 76.835 65.7225) (end 76.835 75.2475) (width 0.5) (layer F.Cu) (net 13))
 (segment (start 74.97815 63.86565) (end 76.835 65.7225) (width 0.5) (layer F.Cu) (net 13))
 (segment (start 70.85065 63.86565) (end 74.97815 63.86565) (width 0.5) (layer F.Cu) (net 13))
 (segment (start 69.85 62.865) (end 70.85065 63.86565) (width 0.5) (layer F.Cu) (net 13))
 (segment (start 69.85 60.96) (end 69.85 62.865) (width 0.5) (layer F.Cu) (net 13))
 (segment (start 76.2 79.93) (end 76.2 81.28) (width 0.5) (layer B.Cu) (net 12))
 (segment (start 76.2 79.5133) (end 76.2 79.93) (width 0.5) (layer B.Cu) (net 12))
 (segment (start 66.0366 69.3499) (end 76.2 79.5133) (width 0.5) (layer B.Cu) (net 12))
 (segment (start 66.0366 67.3066) (end 66.0366 69.3499) (width 0.5) (layer B.Cu) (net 12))
 (segment (start 60.0075 66.675) (end 65.405 66.675) (width 0.5) (layer B.Cu) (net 12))
 (segment (start 65.405 66.675) (end 66.0366 67.3066) (width 0.5) (layer B.Cu) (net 12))
 (segment (start 59.69 66.9925) (end 60.0075 66.675) (width 0.5) (layer B.Cu) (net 12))
 (segment (start 59.69 68.58) (end 59.69 66.9925) (width 0.5) (layer B.Cu) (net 12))
 (segment (start 73.66 81.28) (end 73.66 79.93) (width 0.5) (layer B.Cu) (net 11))
 (segment (start 66.2844 72.5544) (end 73.66 79.93) (width 0.5) (layer B.Cu) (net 11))
 (via (at 66.2844 71.755) (size 1.3) (drill 0.5) (layers F.Cu B.Cu) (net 11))
 (segment (start 66.2844 72.5544) (end 66.2844 71.755) (width 0.5) (layer B.Cu) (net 11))
 (segment (start 66.0204 71.491) (end 66.2844 71.755) (width 0.5) (layer F.Cu) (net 11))
 (segment (start 66.0204 66.0504) (end 66.0204 71.491) (width 0.5) (layer F.Cu) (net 11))
 (segment (start 62.23 62.26) (end 66.0204 66.0504) (width 0.5) (layer F.Cu) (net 11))
 (segment (start 62.23 60.96) (end 62.23 62.26) (width 0.5) (layer F.Cu) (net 11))
 (segment (start 59.69 60.96) (end 59.69 62.26) (width 0.5) (layer F.Cu) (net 26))
 (segment (start 59.69 62.26) (end 49.4522 72.4978) (width 0.5) (layer F.Cu) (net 26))
 (segment (start 49.4522 72.4978) (end 49.4522 81.7713) (width 0.5) (layer F.Cu) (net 26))
 (segment (start 49.4522 81.7713) (end 51.0405 83.3596) (width 0.5) (layer F.Cu) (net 26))
 (segment (start 51.0405 83.3596) (end 93.0904 83.3596) (width 0.5) (layer F.Cu) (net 26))
 (segment (start 96.52 81.28) (end 96.52 82.55) (width 0.5) (layer F.Cu) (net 26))
 (segment (start 96.52 82.55) (end 95.925 83.145) (width 0.5) (layer F.Cu) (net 26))
 (segment (start 95.925 83.145) (end 95.72501 83.34499) (width 0.5) (layer F.Cu) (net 26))
 (segment (start 95.72501 83.34499) (end 93.0904 83.34499) (width 0.5) (layer F.Cu) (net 26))
 (segment (start 57.15 66.675) (end 57.15 68.58) (width 0.5) (layer B.Cu) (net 25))
 (segment (start 99.06 81.28) (end 97.5272 79.7472) (width 0.5) (layer B.Cu) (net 25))
 (segment (start 71.12 66.675) (end 70.1675 65.7225) (width 0.5) (layer B.Cu) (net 25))
 (segment (start 70.1675 65.7225) (end 58.1025 65.7225) (width 0.5) (layer B.Cu) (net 25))
 (segment (start 89.2722 79.7472) (end 85.4075 75.8825) (width 0.5) (layer B.Cu) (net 25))
 (segment (start 85.4075 75.8825) (end 85.4075 72.7209) (width 0.5) (layer B.Cu) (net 25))
 (segment (start 85.4075 72.7209) (end 84.7591 72.0725) (width 0.5) (layer B.Cu) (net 25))
 (segment (start 73.3425 72.7075) (end 71.12 70.485) (width 0.5) (layer B.Cu) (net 25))
 (segment (start 84.7591 72.0725) (end 82.2325 72.0725) (width 0.5) (layer B.Cu) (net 25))
 (segment (start 82.2325 72.0725) (end 81.5975 72.7075) (width 0.5) (layer B.Cu) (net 25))
 (segment (start 71.12 70.485) (end 71.12 66.675) (width 0.5) (layer B.Cu) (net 25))
 (segment (start 97.5272 79.7472) (end 89.2722 79.7472) (width 0.5) (layer B.Cu) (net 25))
 (segment (start 81.5975 72.7075) (end 73.3425 72.7075) (width 0.5) (layer B.Cu) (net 25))
 (segment (start 58.1025 65.7225) (end 57.15 66.675) (width 0.5) (layer B.Cu) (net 25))
 (via (at 74.93 71.4375) (size 1.3) (drill 0.5) (layers F.Cu B.Cu) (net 24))
 (segment (start 73.66 70.1675) (end 74.93 71.4375) (width 0.5) (layer F.Cu) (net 24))
 (segment (start 73.66 66.675) (end 73.66 70.1675) (width 0.5) (layer F.Cu) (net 24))
 (segment (start 72.9144 65.9294) (end 73.66 66.675) (width 0.5) (layer F.Cu) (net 24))
 (segment (start 70.6919 65.9294) (end 72.9144 65.9294) (width 0.5) (layer F.Cu) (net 24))
 (segment (start 67.31 62.5475) (end 70.6919 65.9294) (width 0.5) (layer F.Cu) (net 24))
 (segment (start 67.31 60.96) (end 67.31 62.5475) (width 0.5) (layer F.Cu) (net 24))
 (segment (start 98.7425 78.4225) (end 101.6 81.28) (width 0.5) (layer B.Cu) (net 24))
 (segment (start 86.36 74.6125) (end 90.17 78.4225) (width 0.5) (layer B.Cu) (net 24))
 (segment (start 86.36 72.39) (end 86.36 74.6125) (width 0.5) (layer B.Cu) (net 24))
 (segment (start 84.6885 70.7185) (end 86.36 72.39) (width 0.5) (layer B.Cu) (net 24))
 (segment (start 81.0465 70.7185) (end 84.6885 70.7185) (width 0.5) (layer B.Cu) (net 24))
 (segment (start 80.3275 71.4375) (end 81.0465 70.7185) (width 0.5) (layer B.Cu) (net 24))
 (segment (start 90.17 78.4225) (end 98.7425 78.4225) (width 0.5) (layer B.Cu) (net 24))
 (segment (start 74.93 71.4375) (end 80.3275 71.4375) (width 0.5) (layer B.Cu) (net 24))
 (segment (start 103.505 83.185) (end 104.14 82.55) (width 0.5) (layer B.Cu) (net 23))
 (segment (start 72.39 83.185) (end 103.505 83.185) (width 0.5) (layer B.Cu) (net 23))
 (segment (start 71.77775 82.57275) (end 72.39 83.185) (width 0.5) (layer B.Cu) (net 23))
 (segment (start 104.14 82.55) (end 104.14 81.28) (width 0.5) (layer B.Cu) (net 23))
 (segment (start 71.77775 81.25725) (end 71.77775 82.57275) (width 0.5) (layer B.Cu) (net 23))
 (segment (start 64.77 74.2495) (end 71.77775 81.25725) (width 0.5) (layer B.Cu) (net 23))
 (segment (start 64.77 68.58) (end 64.77 74.2495) (width 0.5) (layer B.Cu) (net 23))
 (segment (start 95.25 59.69) (end 95.25 60.96) (width 0.5) (layer B.Cu) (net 22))
 (segment (start 95.885 59.055) (end 95.25 59.69) (width 0.5) (layer B.Cu) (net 22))
 (segment (start 121.285 59.055) (end 95.885 59.055) (width 0.5) (layer B.Cu) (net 22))
 (segment (start 128.3004 66.0704) (end 121.285 59.055) (width 0.5) (layer B.Cu) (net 22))
 (segment (start 128.3004 82.3166) (end 128.3004 66.0704) (width 0.5) (layer B.Cu) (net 22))
 (segment (start 127.3284 83.2886) (end 128.3004 82.3166) (width 0.5) (layer B.Cu) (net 22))
 (segment (start 107.4186 83.2886) (end 127.3284 83.2886) (width 0.5) (layer B.Cu) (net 22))
 (segment (start 106.68 82.55) (end 107.4186 83.2886) (width 0.5) (layer B.Cu) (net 22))
 (segment (start 106.68 81.28) (end 106.68 82.55) (width 0.5) (layer B.Cu) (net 22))
 (segment (start 109.22 81.28) (end 109.22 79.93) (width 0.5) (layer F.Cu) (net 21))
 (segment (start 87.63 60.96) (end 88.9145 59.6755) (width 0.5) (layer F.Cu) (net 21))
 (segment (start 88.9145 59.6755) (end 98.2776 59.6755) (width 0.5) (layer F.Cu) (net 21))
 (segment (start 98.2776 59.6755) (end 99.06 60.4579) (width 0.5) (layer F.Cu) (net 21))
 (segment (start 99.06 60.4579) (end 99.06 69.77) (width 0.5) (layer F.Cu) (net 21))
 (segment (start 99.06 69.77) (end 109.22 79.93) (width 0.5) (layer F.Cu) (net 21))
 (segment (start 115.601 82.3675) (end 115.3882 82.5803) (width 0.5) (layer B.Cu) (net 20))
 (segment (start 113.0603 82.5803) (end 111.76 81.28) (width 0.5) (layer B.Cu) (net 20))
 (segment (start 115.3882 82.5803) (end 113.0603 82.5803) (width 0.5) (layer B.Cu) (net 20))
 (segment (start 115.601 80.2441) (end 115.601 82.3675) (width 0.5) (layer B.Cu) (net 20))
 (segment (start 110.3272 74.9703) (end 115.601 80.2441) (width 0.5) (layer B.Cu) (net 20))
 (segment (start 97.1953 74.9703) (end 110.3272 74.9703) (width 0.5) (layer B.Cu) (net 20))
 (segment (start 92.71 70.485) (end 97.1953 74.9703) (width 0.5) (layer B.Cu) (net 20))
 (segment (start 92.71 68.58) (end 92.71 70.485) (width 0.5) (layer B.Cu) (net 20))
 (segment (start 85.09 69.5241) (end 85.09 68.58) (width 0.5) (layer B.Cu) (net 19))
 (segment (start 93.0359 77.47) (end 85.09 69.5241) (width 0.5) (layer B.Cu) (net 19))
 (segment (start 110.49 77.47) (end 93.0359 77.47) (width 0.5) (layer B.Cu) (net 19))
 (segment (start 114.3 81.28) (end 110.49 77.47) (width 0.5) (layer B.Cu) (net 19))
 (segment (start 102.87 60.96) (end 102.87 62.26) (width 0.5) (layer F.Cu) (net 28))
 (segment (start 102.87 62.26) (end 119.38 78.77) (width 0.5) (layer F.Cu) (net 28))
 (segment (start 119.38 78.77) (end 119.38 81.28) (width 0.5) (layer F.Cu) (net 28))
 (segment (start 102.87 59.055) (end 102.87 60.96) (width 0.5) (layer F.Cu) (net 28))
 (segment (start 82.55 57.15) (end 100.965 57.15) (width 0.5) (layer F.Cu) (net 28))
 (segment (start 78.74 60.96) (end 82.55 57.15) (width 0.5) (layer F.Cu) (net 28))
 (segment (start 100.965 57.15) (end 102.87 59.055) (width 0.5) (layer F.Cu) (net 28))
 (segment (start 74.93 60.96) (end 78.74 60.96) (width 0.5) (layer F.Cu) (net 28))
 (segment (start 127 81.28) (end 127 79.93) (width 0.5) (layer B.Cu) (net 27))
 (segment (start 127 79.93) (end 126.73 79.66) (width 0.5) (layer B.Cu) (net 27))
 (segment (start 126.73 79.66) (end 126.73 77.47) (width 0.5) (layer B.Cu) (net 27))
 (segment (start 72.39 69.85) (end 72.39 68.58) (width 0.5) (layer B.Cu) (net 27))
 (segment (start 79.0575 70.1675) (end 72.7075 70.1675) (width 0.5) (layer B.Cu) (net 27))
 (segment (start 82.55 66.675) (end 79.0575 70.1675) (width 0.5) (layer B.Cu) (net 27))
 (segment (start 99.695 66.675) (end 82.55 66.675) (width 0.5) (layer B.Cu) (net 27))
 (segment (start 100.33 67.31) (end 99.695 66.675) (width 0.5) (layer B.Cu) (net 27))
 (segment (start 72.7075 70.1675) (end 72.39 69.85) (width 0.5) (layer B.Cu) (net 27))
 (segment (start 100.33 68.58) (end 100.33 67.31) (width 0.5) (layer B.Cu) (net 27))
 (segment (start 109.642 77.892) (end 100.33 68.58) (width 0.5) (layer F.Cu) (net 27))
 (segment (start 116.9331 82.3256) (end 116.9331 80.8694) (width 0.5) (layer F.Cu) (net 27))
 (segment (start 117.7925 83.185) (end 116.9331 82.3256) (width 0.5) (layer F.Cu) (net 27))
 (segment (start 126.365 83.185) (end 117.7925 83.185) (width 0.5) (layer F.Cu) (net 27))
 (segment (start 113.9557 77.892) (end 109.642 77.892) (width 0.5) (layer F.Cu) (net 27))
 (segment (start 116.9331 80.8694) (end 113.9557 77.892) (width 0.5) (layer F.Cu) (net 27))
 (segment (start 127 82.55) (end 126.365 83.185) (width 0.5) (layer F.Cu) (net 27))
 (segment (start 127 81.28) (end 127 82.55) (width 0.5) (layer F.Cu) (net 27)))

